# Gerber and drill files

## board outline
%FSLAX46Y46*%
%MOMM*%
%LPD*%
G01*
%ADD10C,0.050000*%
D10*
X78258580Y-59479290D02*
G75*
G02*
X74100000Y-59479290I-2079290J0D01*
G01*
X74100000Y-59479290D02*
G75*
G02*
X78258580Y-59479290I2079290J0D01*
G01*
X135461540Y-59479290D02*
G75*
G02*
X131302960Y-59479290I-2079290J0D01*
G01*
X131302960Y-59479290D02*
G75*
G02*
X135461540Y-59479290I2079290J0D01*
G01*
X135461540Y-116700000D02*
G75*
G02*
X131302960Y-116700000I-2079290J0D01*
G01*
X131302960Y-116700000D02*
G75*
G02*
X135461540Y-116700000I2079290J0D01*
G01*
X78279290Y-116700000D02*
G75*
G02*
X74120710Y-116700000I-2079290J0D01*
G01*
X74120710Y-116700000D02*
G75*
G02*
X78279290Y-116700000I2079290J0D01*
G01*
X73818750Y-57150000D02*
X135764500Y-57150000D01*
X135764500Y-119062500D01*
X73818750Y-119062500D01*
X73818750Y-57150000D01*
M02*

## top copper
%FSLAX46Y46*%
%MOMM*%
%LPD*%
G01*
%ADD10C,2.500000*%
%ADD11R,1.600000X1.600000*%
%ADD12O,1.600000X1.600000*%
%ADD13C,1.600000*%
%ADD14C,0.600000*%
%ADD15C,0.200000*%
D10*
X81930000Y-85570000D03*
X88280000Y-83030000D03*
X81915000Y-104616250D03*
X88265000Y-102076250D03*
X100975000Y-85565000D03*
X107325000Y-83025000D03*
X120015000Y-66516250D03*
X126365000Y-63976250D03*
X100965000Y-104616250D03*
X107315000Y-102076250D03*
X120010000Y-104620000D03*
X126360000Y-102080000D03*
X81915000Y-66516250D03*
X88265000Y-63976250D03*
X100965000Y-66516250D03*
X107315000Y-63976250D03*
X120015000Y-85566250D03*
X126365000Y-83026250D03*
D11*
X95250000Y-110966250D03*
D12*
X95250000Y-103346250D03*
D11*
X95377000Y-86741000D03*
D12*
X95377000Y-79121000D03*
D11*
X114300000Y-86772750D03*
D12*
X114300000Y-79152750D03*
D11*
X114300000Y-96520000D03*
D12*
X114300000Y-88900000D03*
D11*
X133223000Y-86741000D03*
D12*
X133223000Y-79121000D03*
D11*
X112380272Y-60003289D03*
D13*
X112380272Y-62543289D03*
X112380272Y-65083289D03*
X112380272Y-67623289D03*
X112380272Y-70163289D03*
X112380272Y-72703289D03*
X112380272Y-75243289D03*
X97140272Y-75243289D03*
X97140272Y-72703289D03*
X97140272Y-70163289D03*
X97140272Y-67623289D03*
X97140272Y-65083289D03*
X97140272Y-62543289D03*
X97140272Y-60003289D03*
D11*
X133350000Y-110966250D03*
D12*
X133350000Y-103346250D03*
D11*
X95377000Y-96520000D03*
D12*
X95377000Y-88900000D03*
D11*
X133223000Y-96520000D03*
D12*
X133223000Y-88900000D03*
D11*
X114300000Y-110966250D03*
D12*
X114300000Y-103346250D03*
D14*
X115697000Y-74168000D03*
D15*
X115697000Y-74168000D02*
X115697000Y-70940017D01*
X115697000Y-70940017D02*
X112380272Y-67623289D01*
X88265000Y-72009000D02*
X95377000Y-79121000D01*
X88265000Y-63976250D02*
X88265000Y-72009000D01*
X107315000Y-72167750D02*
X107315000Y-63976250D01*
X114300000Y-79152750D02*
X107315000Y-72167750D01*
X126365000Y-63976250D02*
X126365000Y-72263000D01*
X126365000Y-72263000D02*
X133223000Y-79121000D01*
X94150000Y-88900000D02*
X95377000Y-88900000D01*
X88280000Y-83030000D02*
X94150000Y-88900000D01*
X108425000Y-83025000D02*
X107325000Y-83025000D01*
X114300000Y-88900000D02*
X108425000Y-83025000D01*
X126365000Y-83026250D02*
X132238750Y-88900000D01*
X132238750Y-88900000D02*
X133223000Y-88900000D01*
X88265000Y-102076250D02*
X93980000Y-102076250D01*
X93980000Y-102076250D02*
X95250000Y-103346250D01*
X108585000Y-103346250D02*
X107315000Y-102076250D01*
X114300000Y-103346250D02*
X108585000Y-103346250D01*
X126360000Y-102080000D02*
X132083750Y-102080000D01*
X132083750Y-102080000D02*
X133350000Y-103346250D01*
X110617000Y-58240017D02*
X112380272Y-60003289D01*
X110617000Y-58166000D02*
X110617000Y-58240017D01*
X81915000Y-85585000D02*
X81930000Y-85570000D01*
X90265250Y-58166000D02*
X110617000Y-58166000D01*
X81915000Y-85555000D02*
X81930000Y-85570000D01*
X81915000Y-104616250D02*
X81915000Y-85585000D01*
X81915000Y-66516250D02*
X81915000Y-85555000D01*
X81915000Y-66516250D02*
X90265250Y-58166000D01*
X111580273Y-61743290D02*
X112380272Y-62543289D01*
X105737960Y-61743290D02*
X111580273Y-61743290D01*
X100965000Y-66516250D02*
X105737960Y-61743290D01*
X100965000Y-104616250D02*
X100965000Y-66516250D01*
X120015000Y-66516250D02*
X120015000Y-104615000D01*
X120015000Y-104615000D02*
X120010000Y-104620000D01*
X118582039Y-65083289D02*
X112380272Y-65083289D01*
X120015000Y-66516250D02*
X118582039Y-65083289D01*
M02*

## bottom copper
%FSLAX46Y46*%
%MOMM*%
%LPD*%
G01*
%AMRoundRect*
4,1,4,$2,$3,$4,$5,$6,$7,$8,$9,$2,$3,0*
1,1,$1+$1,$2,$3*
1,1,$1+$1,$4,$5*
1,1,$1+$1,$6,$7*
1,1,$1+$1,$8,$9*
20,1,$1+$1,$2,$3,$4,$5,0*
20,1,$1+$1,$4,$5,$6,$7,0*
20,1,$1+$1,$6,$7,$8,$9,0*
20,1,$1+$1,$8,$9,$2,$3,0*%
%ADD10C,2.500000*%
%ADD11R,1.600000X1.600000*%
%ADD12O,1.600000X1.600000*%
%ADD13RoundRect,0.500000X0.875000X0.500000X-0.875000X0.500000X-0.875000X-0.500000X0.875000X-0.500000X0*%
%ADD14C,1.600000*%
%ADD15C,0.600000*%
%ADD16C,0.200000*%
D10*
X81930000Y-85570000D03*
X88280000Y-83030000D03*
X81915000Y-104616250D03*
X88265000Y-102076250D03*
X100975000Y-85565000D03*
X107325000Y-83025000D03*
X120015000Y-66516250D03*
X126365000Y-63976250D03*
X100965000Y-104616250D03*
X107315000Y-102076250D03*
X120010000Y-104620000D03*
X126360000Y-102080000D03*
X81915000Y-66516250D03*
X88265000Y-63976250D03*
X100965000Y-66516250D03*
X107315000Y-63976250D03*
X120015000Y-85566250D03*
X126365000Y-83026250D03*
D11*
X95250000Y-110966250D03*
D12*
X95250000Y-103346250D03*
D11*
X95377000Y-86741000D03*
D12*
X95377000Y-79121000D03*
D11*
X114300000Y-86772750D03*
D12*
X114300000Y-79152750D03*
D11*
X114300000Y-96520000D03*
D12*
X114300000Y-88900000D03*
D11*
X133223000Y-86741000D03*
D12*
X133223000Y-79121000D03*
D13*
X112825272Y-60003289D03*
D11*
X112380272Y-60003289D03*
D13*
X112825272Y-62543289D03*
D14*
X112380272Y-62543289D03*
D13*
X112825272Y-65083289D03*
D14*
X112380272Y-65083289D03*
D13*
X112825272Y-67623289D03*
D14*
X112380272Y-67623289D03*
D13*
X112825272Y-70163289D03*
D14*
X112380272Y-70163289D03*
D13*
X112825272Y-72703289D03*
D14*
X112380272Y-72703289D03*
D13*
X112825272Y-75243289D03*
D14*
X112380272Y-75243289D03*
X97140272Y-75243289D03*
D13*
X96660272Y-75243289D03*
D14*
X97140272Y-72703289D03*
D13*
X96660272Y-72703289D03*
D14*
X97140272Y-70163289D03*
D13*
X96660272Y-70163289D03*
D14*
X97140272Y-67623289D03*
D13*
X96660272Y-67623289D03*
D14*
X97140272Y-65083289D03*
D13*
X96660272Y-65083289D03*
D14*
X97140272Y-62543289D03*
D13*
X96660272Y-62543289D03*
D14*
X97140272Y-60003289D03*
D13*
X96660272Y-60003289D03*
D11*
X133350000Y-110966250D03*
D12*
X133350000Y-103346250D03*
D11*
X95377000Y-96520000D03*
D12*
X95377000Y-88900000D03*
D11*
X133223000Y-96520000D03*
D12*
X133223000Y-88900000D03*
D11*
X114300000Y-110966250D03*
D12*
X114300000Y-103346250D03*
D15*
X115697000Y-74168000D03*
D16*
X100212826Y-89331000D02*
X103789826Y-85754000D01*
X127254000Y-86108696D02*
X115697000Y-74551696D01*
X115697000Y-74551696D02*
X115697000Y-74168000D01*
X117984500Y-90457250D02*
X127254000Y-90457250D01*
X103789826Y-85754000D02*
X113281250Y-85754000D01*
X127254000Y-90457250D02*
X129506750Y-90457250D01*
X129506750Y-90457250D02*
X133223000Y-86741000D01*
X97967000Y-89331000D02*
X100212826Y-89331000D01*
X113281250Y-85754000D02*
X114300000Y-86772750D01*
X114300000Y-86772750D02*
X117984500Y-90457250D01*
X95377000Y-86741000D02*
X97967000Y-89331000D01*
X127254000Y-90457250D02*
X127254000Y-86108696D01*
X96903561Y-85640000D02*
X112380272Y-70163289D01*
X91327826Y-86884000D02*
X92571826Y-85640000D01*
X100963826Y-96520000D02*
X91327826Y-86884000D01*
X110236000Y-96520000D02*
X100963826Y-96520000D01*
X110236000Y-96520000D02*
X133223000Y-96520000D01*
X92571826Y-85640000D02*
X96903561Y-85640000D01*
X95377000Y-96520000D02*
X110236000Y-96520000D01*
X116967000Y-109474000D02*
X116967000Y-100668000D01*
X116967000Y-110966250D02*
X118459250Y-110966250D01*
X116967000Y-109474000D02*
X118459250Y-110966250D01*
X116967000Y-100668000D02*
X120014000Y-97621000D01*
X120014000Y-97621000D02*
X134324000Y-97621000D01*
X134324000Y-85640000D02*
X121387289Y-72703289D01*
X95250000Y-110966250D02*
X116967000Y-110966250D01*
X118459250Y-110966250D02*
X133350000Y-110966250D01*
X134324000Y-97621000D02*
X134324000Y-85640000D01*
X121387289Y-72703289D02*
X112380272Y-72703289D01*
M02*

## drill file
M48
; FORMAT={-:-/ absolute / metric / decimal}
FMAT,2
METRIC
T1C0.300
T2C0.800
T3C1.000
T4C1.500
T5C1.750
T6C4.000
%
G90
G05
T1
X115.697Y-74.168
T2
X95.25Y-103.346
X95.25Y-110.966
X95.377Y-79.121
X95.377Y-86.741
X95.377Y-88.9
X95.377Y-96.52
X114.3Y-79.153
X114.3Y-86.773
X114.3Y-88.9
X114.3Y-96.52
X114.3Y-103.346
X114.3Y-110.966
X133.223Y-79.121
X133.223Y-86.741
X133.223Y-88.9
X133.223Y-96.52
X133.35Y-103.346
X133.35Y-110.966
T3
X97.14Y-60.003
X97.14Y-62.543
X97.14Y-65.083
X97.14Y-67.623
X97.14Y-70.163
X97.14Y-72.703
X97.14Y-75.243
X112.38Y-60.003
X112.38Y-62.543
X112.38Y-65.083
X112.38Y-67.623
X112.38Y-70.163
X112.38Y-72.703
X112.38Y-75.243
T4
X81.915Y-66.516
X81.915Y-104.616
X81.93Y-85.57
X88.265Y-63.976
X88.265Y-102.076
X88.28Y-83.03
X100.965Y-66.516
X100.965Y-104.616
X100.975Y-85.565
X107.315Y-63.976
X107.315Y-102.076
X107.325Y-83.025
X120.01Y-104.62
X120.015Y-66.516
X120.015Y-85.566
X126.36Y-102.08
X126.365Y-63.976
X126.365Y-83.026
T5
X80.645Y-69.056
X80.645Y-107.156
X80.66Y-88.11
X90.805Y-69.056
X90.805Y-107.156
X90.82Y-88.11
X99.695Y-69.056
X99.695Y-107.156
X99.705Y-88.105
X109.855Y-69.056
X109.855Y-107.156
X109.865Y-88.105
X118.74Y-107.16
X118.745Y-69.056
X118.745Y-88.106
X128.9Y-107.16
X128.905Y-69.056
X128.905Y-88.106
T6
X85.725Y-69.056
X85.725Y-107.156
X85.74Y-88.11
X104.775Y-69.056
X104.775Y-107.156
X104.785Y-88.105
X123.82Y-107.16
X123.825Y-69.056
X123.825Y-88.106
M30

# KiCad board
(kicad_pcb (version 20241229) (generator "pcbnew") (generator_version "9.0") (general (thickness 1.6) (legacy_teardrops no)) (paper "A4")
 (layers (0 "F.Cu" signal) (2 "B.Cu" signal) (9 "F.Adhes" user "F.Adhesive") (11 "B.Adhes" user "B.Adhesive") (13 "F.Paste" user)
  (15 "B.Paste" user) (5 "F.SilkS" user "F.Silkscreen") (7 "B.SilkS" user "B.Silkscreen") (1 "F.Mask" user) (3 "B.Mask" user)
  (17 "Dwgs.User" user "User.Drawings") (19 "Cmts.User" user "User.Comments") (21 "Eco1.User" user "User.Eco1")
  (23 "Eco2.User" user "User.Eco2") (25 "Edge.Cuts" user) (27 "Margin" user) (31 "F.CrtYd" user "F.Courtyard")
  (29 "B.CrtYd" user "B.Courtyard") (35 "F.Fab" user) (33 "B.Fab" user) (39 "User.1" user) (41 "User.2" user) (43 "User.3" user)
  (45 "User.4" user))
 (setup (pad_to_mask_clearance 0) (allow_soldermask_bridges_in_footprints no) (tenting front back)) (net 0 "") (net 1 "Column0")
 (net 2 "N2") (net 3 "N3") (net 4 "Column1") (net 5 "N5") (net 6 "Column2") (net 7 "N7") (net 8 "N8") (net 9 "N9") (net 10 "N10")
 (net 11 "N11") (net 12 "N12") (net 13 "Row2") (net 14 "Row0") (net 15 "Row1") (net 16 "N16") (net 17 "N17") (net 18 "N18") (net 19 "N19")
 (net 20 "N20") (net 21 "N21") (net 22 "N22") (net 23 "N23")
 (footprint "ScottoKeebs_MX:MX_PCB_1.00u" (layer "F.Cu") (at 85.74 88.11)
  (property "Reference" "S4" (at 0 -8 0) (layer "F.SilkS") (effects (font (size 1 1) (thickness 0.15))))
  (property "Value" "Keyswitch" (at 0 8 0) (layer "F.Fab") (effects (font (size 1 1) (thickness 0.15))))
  (pad "" np_thru_hole circle (at -5.08 0) (size 1.75 1.75) (drill 1.75) (layers "*.Cu" "*.Mask"))
  (pad "" np_thru_hole circle (at 0 0) (size 4 4) (drill 4) (layers "*.Cu" "*.Mask"))
  (pad "" np_thru_hole circle (at 5.08 0) (size 1.75 1.75) (drill 1.75) (layers "*.Cu" "*.Mask"))
  (pad "1" thru_hole circle (at -3.81 -2.54) (size 2.5 2.5) (drill 1.5) (layers "*.Cu" "*.Mask") (remove_unused_layers no) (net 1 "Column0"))
  (pad "2" thru_hole circle (at 2.54 -5.08) (size 2.5 2.5) (drill 1.5) (layers "*.Cu" "*.Mask") (remove_unused_layers no) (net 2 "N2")))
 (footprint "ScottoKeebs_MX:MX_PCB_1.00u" (layer "F.Cu") (at 85.725 107.15625)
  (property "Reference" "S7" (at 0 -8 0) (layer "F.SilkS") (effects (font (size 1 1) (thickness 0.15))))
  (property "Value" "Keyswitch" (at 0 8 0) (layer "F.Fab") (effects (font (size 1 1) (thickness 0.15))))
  (pad "" np_thru_hole circle (at -5.08 0) (size 1.75 1.75) (drill 1.75) (layers "*.Cu" "*.Mask"))
  (pad "" np_thru_hole circle (at 0 0) (size 4 4) (drill 4) (layers "*.Cu" "*.Mask"))
  (pad "" np_thru_hole circle (at 5.08 0) (size 1.75 1.75) (drill 1.75) (layers "*.Cu" "*.Mask"))
  (pad "1" thru_hole circle (at -3.81 -2.54) (size 2.5 2.5) (drill 1.5) (layers "*.Cu" "*.Mask") (remove_unused_layers no) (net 1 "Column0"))
  (pad "2" thru_hole circle (at 2.54 -5.08) (size 2.5 2.5) (drill 1.5) (layers "*.Cu" "*.Mask") (remove_unused_layers no) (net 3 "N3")))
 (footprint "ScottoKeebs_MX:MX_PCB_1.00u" (layer "F.Cu") (at 104.785 88.105)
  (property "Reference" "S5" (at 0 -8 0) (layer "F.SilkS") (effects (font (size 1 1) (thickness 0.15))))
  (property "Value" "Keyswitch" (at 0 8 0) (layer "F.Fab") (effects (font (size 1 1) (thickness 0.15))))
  (pad "" np_thru_hole circle (at -5.08 0) (size 1.75 1.75) (drill 1.75) (layers "*.Cu" "*.Mask"))
  (pad "" np_thru_hole circle (at 0 0) (size 4 4) (drill 4) (layers "*.Cu" "*.Mask"))
  (pad "" np_thru_hole circle (at 5.08 0) (size 1.75 1.75) (drill 1.75) (layers "*.Cu" "*.Mask"))
  (pad "1" thru_hole circle (at -3.81 -2.54) (size 2.5 2.5) (drill 1.5) (layers "*.Cu" "*.Mask") (remove_unused_layers no) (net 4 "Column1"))
  (pad "2" thru_hole circle (at 2.54 -5.08) (size 2.5 2.5) (drill 1.5) (layers "*.Cu" "*.Mask") (remove_unused_layers no) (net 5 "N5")))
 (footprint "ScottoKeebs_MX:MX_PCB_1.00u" (layer "F.Cu") (at 123.825 69.05625)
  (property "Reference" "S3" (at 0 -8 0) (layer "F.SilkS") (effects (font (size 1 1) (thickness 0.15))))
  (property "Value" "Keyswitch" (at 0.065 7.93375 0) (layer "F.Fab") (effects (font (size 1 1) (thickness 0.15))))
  (pad "" np_thru_hole circle (at -5.08 0) (size 1.75 1.75) (drill 1.75) (layers "*.Cu" "*.Mask"))
  (pad "" np_thru_hole circle (at 0 0) (size 4 4) (drill 4) (layers "*.Cu" "*.Mask"))
  (pad "" np_thru_hole circle (at 5.08 0) (size 1.75 1.75) (drill 1.75) (layers "*.Cu" "*.Mask"))
  (pad "1" thru_hole circle (at -3.81 -2.54) (size 2.5 2.5) (drill 1.5) (layers "*.Cu" "*.Mask") (remove_unused_layers no) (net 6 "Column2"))
  (pad "2" thru_hole circle (at 2.54 -5.08) (size 2.5 2.5) (drill 1.5) (layers "*.Cu" "*.Mask") (remove_unused_layers no) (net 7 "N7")))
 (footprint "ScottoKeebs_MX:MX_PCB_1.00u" (layer "F.Cu") (at 104.775 107.15625)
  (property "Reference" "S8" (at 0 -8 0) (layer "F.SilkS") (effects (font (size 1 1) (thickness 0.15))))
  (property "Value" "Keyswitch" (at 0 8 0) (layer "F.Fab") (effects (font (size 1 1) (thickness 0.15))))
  (pad "" np_thru_hole circle (at -5.08 0) (size 1.75 1.75) (drill 1.75) (layers "*.Cu" "*.Mask"))
  (pad "" np_thru_hole circle (at 0 0) (size 4 4) (drill 4) (layers "*.Cu" "*.Mask"))
  (pad "" np_thru_hole circle (at 5.08 0) (size 1.75 1.75) (drill 1.75) (layers "*.Cu" "*.Mask"))
  (pad "1" thru_hole circle (at -3.81 -2.54) (size 2.5 2.5) (drill 1.5) (layers "*.Cu" "*.Mask") (remove_unused_layers no) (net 4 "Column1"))
  (pad "2" thru_hole circle (at 2.54 -5.08) (size 2.5 2.5) (drill 1.5) (layers "*.Cu" "*.Mask") (remove_unused_layers no) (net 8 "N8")))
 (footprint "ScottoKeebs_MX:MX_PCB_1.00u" (layer "F.Cu") (at 123.82 107.16)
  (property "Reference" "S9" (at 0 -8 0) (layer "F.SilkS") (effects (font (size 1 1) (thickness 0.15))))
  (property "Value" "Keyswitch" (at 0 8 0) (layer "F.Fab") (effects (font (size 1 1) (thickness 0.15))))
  (pad "" np_thru_hole circle (at -5.08 0) (size 1.75 1.75) (drill 1.75) (layers "*.Cu" "*.Mask"))
  (pad "" np_thru_hole circle (at 0 0) (size 4 4) (drill 4) (layers "*.Cu" "*.Mask"))
  (pad "" np_thru_hole circle (at 5.08 0) (size 1.75 1.75) (drill 1.75) (layers "*.Cu" "*.Mask"))
  (pad "1" thru_hole circle (at -3.81 -2.54) (size 2.5 2.5) (drill 1.5) (layers "*.Cu" "*.Mask") (remove_unused_layers no) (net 6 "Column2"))
  (pad "2" thru_hole circle (at 2.54 -5.08) (size 2.5 2.5) (drill 1.5) (layers "*.Cu" "*.Mask") (remove_unused_layers no) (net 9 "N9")))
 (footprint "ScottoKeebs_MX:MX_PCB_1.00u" (layer "F.Cu") (at 85.725 69.05625)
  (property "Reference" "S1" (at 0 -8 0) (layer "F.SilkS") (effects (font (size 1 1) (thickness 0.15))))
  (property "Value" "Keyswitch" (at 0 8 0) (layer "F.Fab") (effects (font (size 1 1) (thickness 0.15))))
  (pad "" np_thru_hole circle (at -5.08 0) (size 1.75 1.75) (drill 1.75) (layers "*.Cu" "*.Mask"))
  (pad "" np_thru_hole circle (at 0 0) (size 4 4) (drill 4) (layers "*.Cu" "*.Mask"))
  (pad "" np_thru_hole circle (at 5.08 0) (size 1.75 1.75) (drill 1.75) (layers "*.Cu" "*.Mask"))
  (pad "1" thru_hole circle (at -3.81 -2.54) (size 2.5 2.5) (drill 1.5) (layers "*.Cu" "*.Mask") (remove_unused_layers no) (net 1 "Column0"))
  (pad "2" thru_hole circle (at 2.54 -5.08) (size 2.5 2.5) (drill 1.5) (layers "*.Cu" "*.Mask") (remove_unused_layers no) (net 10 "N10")))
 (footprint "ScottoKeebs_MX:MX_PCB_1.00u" (layer "F.Cu") (at 104.775 69.05625)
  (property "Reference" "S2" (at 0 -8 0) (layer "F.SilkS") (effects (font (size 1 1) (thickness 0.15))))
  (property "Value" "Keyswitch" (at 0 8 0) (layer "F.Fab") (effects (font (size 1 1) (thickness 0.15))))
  (pad "" np_thru_hole circle (at -5.08 0) (size 1.75 1.75) (drill 1.75) (layers "*.Cu" "*.Mask"))
  (pad "" np_thru_hole circle (at 0 0) (size 4 4) (drill 4) (layers "*.Cu" "*.Mask"))
  (pad "" np_thru_hole circle (at 5.08 0) (size 1.75 1.75) (drill 1.75) (layers "*.Cu" "*.Mask"))
  (pad "1" thru_hole circle (at -3.81 -2.54) (size 2.5 2.5) (drill 1.5) (layers "*.Cu" "*.Mask") (remove_unused_layers no) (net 4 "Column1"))
  (pad "2" thru_hole circle (at 2.54 -5.08) (size 2.5 2.5) (drill 1.5) (layers "*.Cu" "*.Mask") (remove_unused_layers no) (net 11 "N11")))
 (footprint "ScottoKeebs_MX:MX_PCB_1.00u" (layer "F.Cu") (at 123.825 88.10625)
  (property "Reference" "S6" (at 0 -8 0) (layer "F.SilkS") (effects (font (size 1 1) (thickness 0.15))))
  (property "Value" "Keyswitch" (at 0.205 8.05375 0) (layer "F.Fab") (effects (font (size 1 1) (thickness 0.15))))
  (pad "" np_thru_hole circle (at -5.08 0) (size 1.75 1.75) (drill 1.75) (layers "*.Cu" "*.Mask"))
  (pad "" np_thru_hole circle (at 0 0) (size 4 4) (drill 4) (layers "*.Cu" "*.Mask"))
  (pad "" np_thru_hole circle (at 5.08 0) (size 1.75 1.75) (drill 1.75) (layers "*.Cu" "*.Mask"))
  (pad "1" thru_hole circle (at -3.81 -2.54) (size 2.5 2.5) (drill 1.5) (layers "*.Cu" "*.Mask") (remove_unused_layers no) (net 6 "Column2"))
  (pad "2" thru_hole circle (at 2.54 -5.08) (size 2.5 2.5) (drill 1.5) (layers "*.Cu" "*.Mask") (remove_unused_layers no) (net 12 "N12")))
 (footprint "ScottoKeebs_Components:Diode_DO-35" (layer "B.Cu") (at 95.25 110.96625 90)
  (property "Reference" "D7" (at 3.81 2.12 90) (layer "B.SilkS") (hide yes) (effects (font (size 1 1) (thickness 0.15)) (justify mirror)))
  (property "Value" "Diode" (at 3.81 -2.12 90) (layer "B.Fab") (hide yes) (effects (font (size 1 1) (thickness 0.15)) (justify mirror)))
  (pad "1" thru_hole rect (at 0 0 90) (size 1.6 1.6) (drill 0.8) (layers "*.Cu" "*.Mask") (remove_unused_layers no) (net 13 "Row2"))
  (pad "2" thru_hole oval (at 7.62 0 90) (size 1.6 1.6) (drill 0.8) (layers "*.Cu" "*.Mask") (remove_unused_layers no) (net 3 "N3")))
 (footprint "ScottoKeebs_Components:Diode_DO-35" (layer "B.Cu") (at 95.377 86.741 90)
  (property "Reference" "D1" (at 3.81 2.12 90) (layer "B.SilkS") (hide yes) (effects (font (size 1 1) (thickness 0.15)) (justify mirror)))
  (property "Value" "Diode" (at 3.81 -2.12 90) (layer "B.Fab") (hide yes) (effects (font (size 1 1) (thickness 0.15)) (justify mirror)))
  (pad "1" thru_hole rect (at 0 0 90) (size 1.6 1.6) (drill 0.8) (layers "*.Cu" "*.Mask") (remove_unused_layers no) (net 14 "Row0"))
  (pad "2" thru_hole oval (at 7.62 0 90) (size 1.6 1.6) (drill 0.8) (layers "*.Cu" "*.Mask") (remove_unused_layers no) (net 10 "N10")))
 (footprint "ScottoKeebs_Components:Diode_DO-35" (layer "B.Cu") (at 114.3 86.77275 90)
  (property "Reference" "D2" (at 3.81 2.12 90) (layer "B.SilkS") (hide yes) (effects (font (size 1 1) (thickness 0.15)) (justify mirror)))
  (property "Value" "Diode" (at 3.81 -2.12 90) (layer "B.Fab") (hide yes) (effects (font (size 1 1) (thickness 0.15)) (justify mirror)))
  (pad "1" thru_hole rect (at 0 0 90) (size 1.6 1.6) (drill 0.8) (layers "*.Cu" "*.Mask") (remove_unused_layers no) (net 14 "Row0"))
  (pad "2" thru_hole oval (at 7.62 0 90) (size 1.6 1.6) (drill 0.8) (layers "*.Cu" "*.Mask") (remove_unused_layers no) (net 11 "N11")))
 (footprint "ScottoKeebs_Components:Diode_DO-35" (layer "B.Cu") (at 114.3 96.52 90)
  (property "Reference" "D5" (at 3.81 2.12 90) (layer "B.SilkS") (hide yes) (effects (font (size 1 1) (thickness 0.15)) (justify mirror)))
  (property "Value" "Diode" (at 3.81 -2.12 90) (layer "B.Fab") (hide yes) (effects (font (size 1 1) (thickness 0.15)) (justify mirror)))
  (pad "1" thru_hole rect (at 0 0 90) (size 1.6 1.6) (drill 0.8) (layers "*.Cu" "*.Mask") (remove_unused_layers no) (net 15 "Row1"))
  (pad "2" thru_hole oval (at 7.62 0 90) (size 1.6 1.6) (drill 0.8) (layers "*.Cu" "*.Mask") (remove_unused_layers no) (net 5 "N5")))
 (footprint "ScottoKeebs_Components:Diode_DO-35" (layer "B.Cu") (at 133.223 86.741 90)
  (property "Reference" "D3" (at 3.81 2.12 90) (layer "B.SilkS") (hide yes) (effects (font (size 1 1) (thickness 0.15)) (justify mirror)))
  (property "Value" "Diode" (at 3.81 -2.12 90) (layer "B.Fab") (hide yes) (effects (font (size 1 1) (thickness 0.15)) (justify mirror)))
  (pad "1" thru_hole rect (at 0 0 90) (size 1.6 1.6) (drill 0.8) (layers "*.Cu" "*.Mask") (remove_unused_layers no) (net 14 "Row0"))
  (pad "2" thru_hole oval (at 7.62 0 90) (size 1.6 1.6) (drill 0.8) (layers "*.Cu" "*.Mask") (remove_unused_layers no) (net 7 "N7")))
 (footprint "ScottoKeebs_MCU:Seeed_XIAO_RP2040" (layer "B.Cu") (at 104.760272 67.623289 180)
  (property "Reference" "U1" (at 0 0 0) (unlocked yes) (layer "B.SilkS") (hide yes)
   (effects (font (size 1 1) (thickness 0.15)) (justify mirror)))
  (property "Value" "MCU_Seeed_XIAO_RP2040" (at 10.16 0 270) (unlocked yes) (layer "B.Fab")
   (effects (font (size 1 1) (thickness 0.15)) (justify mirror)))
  (pad "1" smd roundrect (at -8.065 7.62 180) (size 2.75 2) (layers "B.Cu" "B.Mask" "B.Paste") (roundrect_rratio 0.25) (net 1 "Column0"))
  (pad "1" thru_hole rect (at -7.62 7.62 90) (size 1.6 1.6) (drill 1) (layers "*.Cu" "*.Mask") (remove_unused_layers no) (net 1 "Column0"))
  (pad "2" smd roundrect (at -8.065 5.08 180) (size 2.75 2) (layers "B.Cu" "B.Mask" "B.Paste") (roundrect_rratio 0.25) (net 4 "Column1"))
  (pad "2" thru_hole circle (at -7.62 5.08 90) (size 1.6 1.6) (drill 1) (layers "*.Cu" "*.Mask") (remove_unused_layers no) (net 4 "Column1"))
  (pad "3" smd roundrect (at -8.065 2.54 180) (size 2.75 2) (layers "B.Cu" "B.Mask" "B.Paste") (roundrect_rratio 0.25) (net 6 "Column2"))
  (pad "3" thru_hole circle (at -7.62 2.54 90) (size 1.6 1.6) (drill 1) (layers "*.Cu" "*.Mask") (remove_unused_layers no) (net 6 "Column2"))
  (pad "4" smd roundrect (at -8.065 0 180) (size 2.75 2) (layers "B.Cu" "B.Mask" "B.Paste") (roundrect_rratio 0.25) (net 14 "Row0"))
  (pad "4" thru_hole circle (at -7.62 0 90) (size 1.6 1.6) (drill 1) (layers "*.Cu" "*.Mask") (remove_unused_layers no) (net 14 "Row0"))
  (pad "5" smd roundrect (at -8.065 -2.54 180) (size 2.75 2) (layers "B.Cu" "B.Mask" "B.Paste") (roundrect_rratio 0.25) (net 15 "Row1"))
  (pad "5" thru_hole circle (at -7.62 -2.54 90) (size 1.6 1.6) (drill 1) (layers "*.Cu" "*.Mask") (remove_unused_layers no) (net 15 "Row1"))
  (pad "6" smd roundrect (at -8.065 -5.08 180) (size 2.75 2) (layers "B.Cu" "B.Mask" "B.Paste") (roundrect_rratio 0.25) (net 13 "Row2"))
  (pad "6" thru_hole circle (at -7.62 -5.08 90) (size 1.6 1.6) (drill 1) (layers "*.Cu" "*.Mask") (remove_unused_layers no) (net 13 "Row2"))
  (pad "7" smd roundrect (at -8.065 -7.62 180) (size 2.75 2) (layers "B.Cu" "B.Mask" "B.Paste") (roundrect_rratio 0.25) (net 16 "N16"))
  (pad "7" thru_hole circle (at -7.62 -7.62 90) (size 1.6 1.6) (drill 1) (layers "*.Cu" "*.Mask") (remove_unused_layers no) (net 16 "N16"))
  (pad "8" thru_hole circle (at 7.62 -7.62 90) (size 1.6 1.6) (drill 1) (layers "*.Cu" "*.Mask") (remove_unused_layers no) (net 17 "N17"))
  (pad "8" smd roundrect (at 8.1 -7.62 180) (size 2.75 2) (layers "B.Cu" "B.Mask" "B.Paste") (roundrect_rratio 0.25) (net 17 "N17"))
  (pad "9" thru_hole circle (at 7.62 -5.08 90) (size 1.6 1.6) (drill 1) (layers "*.Cu" "*.Mask") (remove_unused_layers no) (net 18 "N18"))
  (pad "9" smd roundrect (at 8.1 -5.08 180) (size 2.75 2) (layers "B.Cu" "B.Mask" "B.Paste") (roundrect_rratio 0.25) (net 18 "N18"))
  (pad "10" thru_hole circle (at 7.62 -2.54 90) (size 1.6 1.6) (drill 1) (layers "*.Cu" "*.Mask") (remove_unused_layers no) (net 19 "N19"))
  (pad "10" smd roundrect (at 8.1 -2.54 180) (size 2.75 2) (layers "B.Cu" "B.Mask" "B.Paste") (roundrect_rratio 0.25) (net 19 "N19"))
  (pad "11" thru_hole circle (at 7.62 0 90) (size 1.6 1.6) (drill 1) (layers "*.Cu" "*.Mask") (remove_unused_layers no) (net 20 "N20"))
  (pad "11" smd roundrect (at 8.1 0 180) (size 2.75 2) (layers "B.Cu" "B.Mask" "B.Paste") (roundrect_rratio 0.25) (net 20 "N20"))
  (pad "12" thru_hole circle (at 7.62 2.54 90) (size 1.6 1.6) (drill 1) (layers "*.Cu" "*.Mask") (remove_unused_layers no) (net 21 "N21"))
  (pad "12" smd roundrect (at 8.1 2.54 180) (size 2.75 2) (layers "B.Cu" "B.Mask" "B.Paste") (roundrect_rratio 0.25) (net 21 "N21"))
  (pad "13" thru_hole circle (at 7.62 5.08 90) (size 1.6 1.6) (drill 1) (layers "*.Cu" "*.Mask") (remove_unused_layers no) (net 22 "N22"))
  (pad "13" smd roundrect (at 8.1 5.08 180) (size 2.75 2) (layers "B.Cu" "B.Mask" "B.Paste") (roundrect_rratio 0.25) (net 22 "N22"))
  (pad "14" thru_hole circle (at 7.62 7.62 90) (size 1.6 1.6) (drill 1) (layers "*.Cu" "*.Mask") (remove_unused_layers no) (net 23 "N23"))
  (pad "14" smd roundrect (at 8.1 7.62 180) (size 2.75 2) (layers "B.Cu" "B.Mask" "B.Paste") (roundrect_rratio 0.25) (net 23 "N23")))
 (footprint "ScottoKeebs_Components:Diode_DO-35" (layer "B.Cu") (at 133.35 110.96625 90)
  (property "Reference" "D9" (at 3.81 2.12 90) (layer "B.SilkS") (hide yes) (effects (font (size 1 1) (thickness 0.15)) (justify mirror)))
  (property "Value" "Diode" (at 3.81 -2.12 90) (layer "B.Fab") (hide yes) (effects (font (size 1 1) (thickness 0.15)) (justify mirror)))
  (pad "1" thru_hole rect (at 0 0 90) (size 1.6 1.6) (drill 0.8) (layers "*.Cu" "*.Mask") (remove_unused_layers no) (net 13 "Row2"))
  (pad "2" thru_hole oval (at 7.62 0 90) (size 1.6 1.6) (drill 0.8) (layers "*.Cu" "*.Mask") (remove_unused_layers no) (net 9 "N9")))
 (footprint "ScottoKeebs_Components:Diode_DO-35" (layer "B.Cu") (at 95.377 96.52 90)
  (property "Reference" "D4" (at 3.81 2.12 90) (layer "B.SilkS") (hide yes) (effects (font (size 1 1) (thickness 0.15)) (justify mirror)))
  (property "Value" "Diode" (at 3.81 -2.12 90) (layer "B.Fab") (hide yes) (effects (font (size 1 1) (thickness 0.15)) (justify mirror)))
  (pad "1" thru_hole rect (at 0 0 90) (size 1.6 1.6) (drill 0.8) (layers "*.Cu" "*.Mask") (remove_unused_layers no) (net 15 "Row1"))
  (pad "2" thru_hole oval (at 7.62 0 90) (size 1.6 1.6) (drill 0.8) (layers "*.Cu" "*.Mask") (remove_unused_layers no) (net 2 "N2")))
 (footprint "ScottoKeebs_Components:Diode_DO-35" (layer "B.Cu") (at 133.223 96.52 90)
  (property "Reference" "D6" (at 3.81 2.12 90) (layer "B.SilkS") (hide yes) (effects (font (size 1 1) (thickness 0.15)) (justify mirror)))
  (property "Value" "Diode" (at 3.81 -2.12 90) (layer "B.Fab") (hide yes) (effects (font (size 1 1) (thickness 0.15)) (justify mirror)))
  (pad "1" thru_hole rect (at 0 0 90) (size 1.6 1.6) (drill 0.8) (layers "*.Cu" "*.Mask") (remove_unused_layers no) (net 15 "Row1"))
  (pad "2" thru_hole oval (at 7.62 0 90) (size 1.6 1.6) (drill 0.8) (layers "*.Cu" "*.Mask") (remove_unused_layers no) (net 12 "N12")))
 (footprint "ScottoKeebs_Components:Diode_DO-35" (layer "B.Cu") (at 114.3 110.96625 90)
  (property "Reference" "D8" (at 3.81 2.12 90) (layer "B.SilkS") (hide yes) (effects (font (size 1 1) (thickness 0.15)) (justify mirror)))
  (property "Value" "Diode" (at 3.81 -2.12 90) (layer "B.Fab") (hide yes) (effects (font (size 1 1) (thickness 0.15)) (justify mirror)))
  (pad "1" thru_hole rect (at 0 0 90) (size 1.6 1.6) (drill 0.8) (layers "*.Cu" "*.Mask") (remove_unused_layers no) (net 13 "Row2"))
  (pad "2" thru_hole oval (at 7.62 0 90) (size 1.6 1.6) (drill 0.8) (layers "*.Cu" "*.Mask") (remove_unused_layers no) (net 8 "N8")))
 (gr_circle (center 76.17929 59.47929) (end 77.64957 60.94957) (stroke (width 0.05) (type default)) (fill no) (layer "Edge.Cuts"))
 (gr_circle (center 133.38225 59.47929) (end 134.85253 60.94957) (stroke (width 0.05) (type default)) (fill no) (layer "Edge.Cuts"))
 (gr_circle (center 133.38225 116.7) (end 134.85253 118.17028) (stroke (width 0.05) (type default)) (fill no) (layer "Edge.Cuts"))
 (gr_circle (center 76.2 116.7) (end 77.67028 118.17028) (stroke (width 0.05) (type default)) (fill no) (layer "Edge.Cuts"))
 (gr_rect (start 73.81875 57.15) (end 135.7645 119.0625) (stroke (width 0.05) (type default)) (fill no) (layer "Edge.Cuts"))
 (segment (start 115.697 74.168) (end 115.697 70.940017) (width 0.2) (layer "F.Cu") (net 14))
 (segment (start 115.697 70.940017) (end 112.380272 67.623289) (width 0.2) (layer "F.Cu") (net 14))
 (via (at 115.697 74.168) (size 0.6) (drill 0.3) (layers "F.Cu" "B.Cu") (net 14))
 (segment (start 100.212826 89.331) (end 103.789826 85.754) (width 0.2) (layer "B.Cu") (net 14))
 (segment (start 127.254 86.108696) (end 115.697 74.551696) (width 0.2) (layer "B.Cu") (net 14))
 (segment (start 115.697 74.551696) (end 115.697 74.168) (width 0.2) (layer "B.Cu") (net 14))
 (segment (start 117.9845 90.45725) (end 127.254 90.45725) (width 0.2) (layer "B.Cu") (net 14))
 (segment (start 103.789826 85.754) (end 113.28125 85.754) (width 0.2) (layer "B.Cu") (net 14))
 (segment (start 127.254 90.45725) (end 129.50675 90.45725) (width 0.2) (layer "B.Cu") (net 14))
 (segment (start 129.50675 90.45725) (end 133.223 86.741) (width 0.2) (layer "B.Cu") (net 14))
 (segment (start 97.967 89.331) (end 100.212826 89.331) (width 0.2) (layer "B.Cu") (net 14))
 (segment (start 113.28125 85.754) (end 114.3 86.77275) (width 0.2) (layer "B.Cu") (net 14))
 (segment (start 114.3 86.77275) (end 117.9845 90.45725) (width 0.2) (layer "B.Cu") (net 14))
 (segment (start 95.377 86.741) (end 97.967 89.331) (width 0.2) (layer "B.Cu") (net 14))
 (segment (start 127.254 90.45725) (end 127.254 86.108696) (width 0.2) (layer "B.Cu") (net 14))
 (segment (start 88.265 72.009) (end 95.377 79.121) (width 0.2) (layer "F.Cu") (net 10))
 (segment (start 88.265 63.97625) (end 88.265 72.009) (width 0.2) (layer "F.Cu") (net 10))
 (segment (start 107.315 72.16775) (end 107.315 63.97625) (width 0.2) (layer "F.Cu") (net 11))
 (segment (start 114.3 79.15275) (end 107.315 72.16775) (width 0.2) (layer "F.Cu") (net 11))
 (segment (start 126.365 63.97625) (end 126.365 72.263) (width 0.2) (layer "F.Cu") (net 7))
 (segment (start 126.365 72.263) (end 133.223 79.121) (width 0.2) (layer "F.Cu") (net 7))
 (segment (start 94.15 88.9) (end 95.377 88.9) (width 0.2) (layer "F.Cu") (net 2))
 (segment (start 88.28 83.03) (end 94.15 88.9) (width 0.2) (layer "F.Cu") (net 2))
 (segment (start 96.903561 85.64) (end 112.380272 70.163289) (width 0.2) (layer "B.Cu") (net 15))
 (segment (start 91.327826 86.884) (end 92.571826 85.64) (width 0.2) (layer "B.Cu") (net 15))
 (segment (start 100.963826 96.52) (end 91.327826 86.884) (width 0.2) (layer "B.Cu") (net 15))
 (segment (start 110.236 96.52) (end 100.963826 96.52) (width 0.2) (layer "B.Cu") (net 15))
 (segment (start 110.236 96.52) (end 133.223 96.52) (width 0.2) (layer "B.Cu") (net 15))
 (segment (start 92.571826 85.64) (end 96.903561 85.64) (width 0.2) (layer "B.Cu") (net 15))
 (segment (start 95.377 96.52) (end 110.236 96.52) (width 0.2) (layer "B.Cu") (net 15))
 (segment (start 108.425 83.025) (end 107.325 83.025) (width 0.2) (layer "F.Cu") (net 5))
 (segment (start 114.3 88.9) (end 108.425 83.025) (width 0.2) (layer "F.Cu") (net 5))
 (segment (start 126.365 83.02625) (end 132.23875 88.9) (width 0.2) (layer "F.Cu") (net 12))
 (segment (start 132.23875 88.9) (end 133.223 88.9) (width 0.2) (layer "F.Cu") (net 12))
 (segment (start 116.967 109.474) (end 116.967 100.668) (width 0.2) (layer "B.Cu") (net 13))
 (segment (start 116.967 110.96625) (end 118.45925 110.96625) (width 0.2) (layer "B.Cu") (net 13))
 (segment (start 116.967 109.474) (end 118.45925 110.96625) (width 0.2) (layer "B.Cu") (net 13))
 (segment (start 116.967 100.668) (end 120.014 97.621) (width 0.2) (layer "B.Cu") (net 13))
 (segment (start 120.014 97.621) (end 134.324 97.621) (width 0.2) (layer "B.Cu") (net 13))
 (segment (start 134.324 85.64) (end 121.387289 72.703289) (width 0.2) (layer "B.Cu") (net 13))
 (segment (start 95.25 110.96625) (end 116.967 110.96625) (width 0.2) (layer "B.Cu") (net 13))
 (segment (start 118.45925 110.96625) (end 133.35 110.96625) (width 0.2) (layer "B.Cu") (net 13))
 (segment (start 134.324 97.621) (end 134.324 85.64) (width 0.2) (layer "B.Cu") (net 13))
 (segment (start 121.387289 72.703289) (end 112.380272 72.703289) (width 0.2) (layer "B.Cu") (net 13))
 (segment (start 88.265 102.07625) (end 93.98 102.07625) (width 0.2) (layer "F.Cu") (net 3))
 (segment (start 93.98 102.07625) (end 95.25 103.34625) (width 0.2) (layer "F.Cu") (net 3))
 (segment (start 108.585 103.34625) (end 107.315 102.07625) (width 0.2) (layer "F.Cu") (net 8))
 (segment (start 114.3 103.34625) (end 108.585 103.34625) (width 0.2) (layer "F.Cu") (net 8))
 (segment (start 126.36 102.08) (end 132.08375 102.08) (width 0.2) (layer "F.Cu") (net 9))
 (segment (start 132.08375 102.08) (end 133.35 103.34625) (width 0.2) (layer "F.Cu") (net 9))
 (segment (start 110.617 58.240017) (end 112.380272 60.003289) (width 0.2) (layer "F.Cu") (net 1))
 (segment (start 110.617 58.166) (end 110.617 58.240017) (width 0.2) (layer "F.Cu") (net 1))
 (segment (start 81.915 85.585) (end 81.93 85.57) (width 0.2) (layer "F.Cu") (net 1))
 (segment (start 90.26525 58.166) (end 110.617 58.166) (width 0.2) (layer "F.Cu") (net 1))
 (segment (start 81.915 85.555) (end 81.93 85.57) (width 0.2) (layer "F.Cu") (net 1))
 (segment (start 81.915 104.61625) (end 81.915 85.585) (width 0.2) (layer "F.Cu") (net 1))
 (segment (start 81.915 66.51625) (end 81.915 85.555) (width 0.2) (layer "F.Cu") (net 1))
 (segment (start 81.915 66.51625) (end 90.26525 58.166) (width 0.2) (layer "F.Cu") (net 1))
 (segment (start 111.580273 61.74329) (end 112.380272 62.543289) (width 0.2) (layer "F.Cu") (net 4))
 (segment (start 105.73796 61.74329) (end 111.580273 61.74329) (width 0.2) (layer "F.Cu") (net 4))
 (segment (start 100.965 66.51625) (end 105.73796 61.74329) (width 0.2) (layer "F.Cu") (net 4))
 (segment (start 100.965 104.61625) (end 100.965 66.51625) (width 0.2) (layer "F.Cu") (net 4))
 (segment (start 120.015 66.51625) (end 120.015 104.615) (width 0.2) (layer "F.Cu") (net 6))
 (segment (start 120.015 104.615) (end 120.01 104.62) (width 0.2) (layer "F.Cu") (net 6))
 (segment (start 118.582039 65.083289) (end 112.380272 65.083289) (width 0.2) (layer "F.Cu") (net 6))
 (segment (start 120.015 66.51625) (end 118.582039 65.083289) (width 0.2) (layer "F.Cu") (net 6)))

